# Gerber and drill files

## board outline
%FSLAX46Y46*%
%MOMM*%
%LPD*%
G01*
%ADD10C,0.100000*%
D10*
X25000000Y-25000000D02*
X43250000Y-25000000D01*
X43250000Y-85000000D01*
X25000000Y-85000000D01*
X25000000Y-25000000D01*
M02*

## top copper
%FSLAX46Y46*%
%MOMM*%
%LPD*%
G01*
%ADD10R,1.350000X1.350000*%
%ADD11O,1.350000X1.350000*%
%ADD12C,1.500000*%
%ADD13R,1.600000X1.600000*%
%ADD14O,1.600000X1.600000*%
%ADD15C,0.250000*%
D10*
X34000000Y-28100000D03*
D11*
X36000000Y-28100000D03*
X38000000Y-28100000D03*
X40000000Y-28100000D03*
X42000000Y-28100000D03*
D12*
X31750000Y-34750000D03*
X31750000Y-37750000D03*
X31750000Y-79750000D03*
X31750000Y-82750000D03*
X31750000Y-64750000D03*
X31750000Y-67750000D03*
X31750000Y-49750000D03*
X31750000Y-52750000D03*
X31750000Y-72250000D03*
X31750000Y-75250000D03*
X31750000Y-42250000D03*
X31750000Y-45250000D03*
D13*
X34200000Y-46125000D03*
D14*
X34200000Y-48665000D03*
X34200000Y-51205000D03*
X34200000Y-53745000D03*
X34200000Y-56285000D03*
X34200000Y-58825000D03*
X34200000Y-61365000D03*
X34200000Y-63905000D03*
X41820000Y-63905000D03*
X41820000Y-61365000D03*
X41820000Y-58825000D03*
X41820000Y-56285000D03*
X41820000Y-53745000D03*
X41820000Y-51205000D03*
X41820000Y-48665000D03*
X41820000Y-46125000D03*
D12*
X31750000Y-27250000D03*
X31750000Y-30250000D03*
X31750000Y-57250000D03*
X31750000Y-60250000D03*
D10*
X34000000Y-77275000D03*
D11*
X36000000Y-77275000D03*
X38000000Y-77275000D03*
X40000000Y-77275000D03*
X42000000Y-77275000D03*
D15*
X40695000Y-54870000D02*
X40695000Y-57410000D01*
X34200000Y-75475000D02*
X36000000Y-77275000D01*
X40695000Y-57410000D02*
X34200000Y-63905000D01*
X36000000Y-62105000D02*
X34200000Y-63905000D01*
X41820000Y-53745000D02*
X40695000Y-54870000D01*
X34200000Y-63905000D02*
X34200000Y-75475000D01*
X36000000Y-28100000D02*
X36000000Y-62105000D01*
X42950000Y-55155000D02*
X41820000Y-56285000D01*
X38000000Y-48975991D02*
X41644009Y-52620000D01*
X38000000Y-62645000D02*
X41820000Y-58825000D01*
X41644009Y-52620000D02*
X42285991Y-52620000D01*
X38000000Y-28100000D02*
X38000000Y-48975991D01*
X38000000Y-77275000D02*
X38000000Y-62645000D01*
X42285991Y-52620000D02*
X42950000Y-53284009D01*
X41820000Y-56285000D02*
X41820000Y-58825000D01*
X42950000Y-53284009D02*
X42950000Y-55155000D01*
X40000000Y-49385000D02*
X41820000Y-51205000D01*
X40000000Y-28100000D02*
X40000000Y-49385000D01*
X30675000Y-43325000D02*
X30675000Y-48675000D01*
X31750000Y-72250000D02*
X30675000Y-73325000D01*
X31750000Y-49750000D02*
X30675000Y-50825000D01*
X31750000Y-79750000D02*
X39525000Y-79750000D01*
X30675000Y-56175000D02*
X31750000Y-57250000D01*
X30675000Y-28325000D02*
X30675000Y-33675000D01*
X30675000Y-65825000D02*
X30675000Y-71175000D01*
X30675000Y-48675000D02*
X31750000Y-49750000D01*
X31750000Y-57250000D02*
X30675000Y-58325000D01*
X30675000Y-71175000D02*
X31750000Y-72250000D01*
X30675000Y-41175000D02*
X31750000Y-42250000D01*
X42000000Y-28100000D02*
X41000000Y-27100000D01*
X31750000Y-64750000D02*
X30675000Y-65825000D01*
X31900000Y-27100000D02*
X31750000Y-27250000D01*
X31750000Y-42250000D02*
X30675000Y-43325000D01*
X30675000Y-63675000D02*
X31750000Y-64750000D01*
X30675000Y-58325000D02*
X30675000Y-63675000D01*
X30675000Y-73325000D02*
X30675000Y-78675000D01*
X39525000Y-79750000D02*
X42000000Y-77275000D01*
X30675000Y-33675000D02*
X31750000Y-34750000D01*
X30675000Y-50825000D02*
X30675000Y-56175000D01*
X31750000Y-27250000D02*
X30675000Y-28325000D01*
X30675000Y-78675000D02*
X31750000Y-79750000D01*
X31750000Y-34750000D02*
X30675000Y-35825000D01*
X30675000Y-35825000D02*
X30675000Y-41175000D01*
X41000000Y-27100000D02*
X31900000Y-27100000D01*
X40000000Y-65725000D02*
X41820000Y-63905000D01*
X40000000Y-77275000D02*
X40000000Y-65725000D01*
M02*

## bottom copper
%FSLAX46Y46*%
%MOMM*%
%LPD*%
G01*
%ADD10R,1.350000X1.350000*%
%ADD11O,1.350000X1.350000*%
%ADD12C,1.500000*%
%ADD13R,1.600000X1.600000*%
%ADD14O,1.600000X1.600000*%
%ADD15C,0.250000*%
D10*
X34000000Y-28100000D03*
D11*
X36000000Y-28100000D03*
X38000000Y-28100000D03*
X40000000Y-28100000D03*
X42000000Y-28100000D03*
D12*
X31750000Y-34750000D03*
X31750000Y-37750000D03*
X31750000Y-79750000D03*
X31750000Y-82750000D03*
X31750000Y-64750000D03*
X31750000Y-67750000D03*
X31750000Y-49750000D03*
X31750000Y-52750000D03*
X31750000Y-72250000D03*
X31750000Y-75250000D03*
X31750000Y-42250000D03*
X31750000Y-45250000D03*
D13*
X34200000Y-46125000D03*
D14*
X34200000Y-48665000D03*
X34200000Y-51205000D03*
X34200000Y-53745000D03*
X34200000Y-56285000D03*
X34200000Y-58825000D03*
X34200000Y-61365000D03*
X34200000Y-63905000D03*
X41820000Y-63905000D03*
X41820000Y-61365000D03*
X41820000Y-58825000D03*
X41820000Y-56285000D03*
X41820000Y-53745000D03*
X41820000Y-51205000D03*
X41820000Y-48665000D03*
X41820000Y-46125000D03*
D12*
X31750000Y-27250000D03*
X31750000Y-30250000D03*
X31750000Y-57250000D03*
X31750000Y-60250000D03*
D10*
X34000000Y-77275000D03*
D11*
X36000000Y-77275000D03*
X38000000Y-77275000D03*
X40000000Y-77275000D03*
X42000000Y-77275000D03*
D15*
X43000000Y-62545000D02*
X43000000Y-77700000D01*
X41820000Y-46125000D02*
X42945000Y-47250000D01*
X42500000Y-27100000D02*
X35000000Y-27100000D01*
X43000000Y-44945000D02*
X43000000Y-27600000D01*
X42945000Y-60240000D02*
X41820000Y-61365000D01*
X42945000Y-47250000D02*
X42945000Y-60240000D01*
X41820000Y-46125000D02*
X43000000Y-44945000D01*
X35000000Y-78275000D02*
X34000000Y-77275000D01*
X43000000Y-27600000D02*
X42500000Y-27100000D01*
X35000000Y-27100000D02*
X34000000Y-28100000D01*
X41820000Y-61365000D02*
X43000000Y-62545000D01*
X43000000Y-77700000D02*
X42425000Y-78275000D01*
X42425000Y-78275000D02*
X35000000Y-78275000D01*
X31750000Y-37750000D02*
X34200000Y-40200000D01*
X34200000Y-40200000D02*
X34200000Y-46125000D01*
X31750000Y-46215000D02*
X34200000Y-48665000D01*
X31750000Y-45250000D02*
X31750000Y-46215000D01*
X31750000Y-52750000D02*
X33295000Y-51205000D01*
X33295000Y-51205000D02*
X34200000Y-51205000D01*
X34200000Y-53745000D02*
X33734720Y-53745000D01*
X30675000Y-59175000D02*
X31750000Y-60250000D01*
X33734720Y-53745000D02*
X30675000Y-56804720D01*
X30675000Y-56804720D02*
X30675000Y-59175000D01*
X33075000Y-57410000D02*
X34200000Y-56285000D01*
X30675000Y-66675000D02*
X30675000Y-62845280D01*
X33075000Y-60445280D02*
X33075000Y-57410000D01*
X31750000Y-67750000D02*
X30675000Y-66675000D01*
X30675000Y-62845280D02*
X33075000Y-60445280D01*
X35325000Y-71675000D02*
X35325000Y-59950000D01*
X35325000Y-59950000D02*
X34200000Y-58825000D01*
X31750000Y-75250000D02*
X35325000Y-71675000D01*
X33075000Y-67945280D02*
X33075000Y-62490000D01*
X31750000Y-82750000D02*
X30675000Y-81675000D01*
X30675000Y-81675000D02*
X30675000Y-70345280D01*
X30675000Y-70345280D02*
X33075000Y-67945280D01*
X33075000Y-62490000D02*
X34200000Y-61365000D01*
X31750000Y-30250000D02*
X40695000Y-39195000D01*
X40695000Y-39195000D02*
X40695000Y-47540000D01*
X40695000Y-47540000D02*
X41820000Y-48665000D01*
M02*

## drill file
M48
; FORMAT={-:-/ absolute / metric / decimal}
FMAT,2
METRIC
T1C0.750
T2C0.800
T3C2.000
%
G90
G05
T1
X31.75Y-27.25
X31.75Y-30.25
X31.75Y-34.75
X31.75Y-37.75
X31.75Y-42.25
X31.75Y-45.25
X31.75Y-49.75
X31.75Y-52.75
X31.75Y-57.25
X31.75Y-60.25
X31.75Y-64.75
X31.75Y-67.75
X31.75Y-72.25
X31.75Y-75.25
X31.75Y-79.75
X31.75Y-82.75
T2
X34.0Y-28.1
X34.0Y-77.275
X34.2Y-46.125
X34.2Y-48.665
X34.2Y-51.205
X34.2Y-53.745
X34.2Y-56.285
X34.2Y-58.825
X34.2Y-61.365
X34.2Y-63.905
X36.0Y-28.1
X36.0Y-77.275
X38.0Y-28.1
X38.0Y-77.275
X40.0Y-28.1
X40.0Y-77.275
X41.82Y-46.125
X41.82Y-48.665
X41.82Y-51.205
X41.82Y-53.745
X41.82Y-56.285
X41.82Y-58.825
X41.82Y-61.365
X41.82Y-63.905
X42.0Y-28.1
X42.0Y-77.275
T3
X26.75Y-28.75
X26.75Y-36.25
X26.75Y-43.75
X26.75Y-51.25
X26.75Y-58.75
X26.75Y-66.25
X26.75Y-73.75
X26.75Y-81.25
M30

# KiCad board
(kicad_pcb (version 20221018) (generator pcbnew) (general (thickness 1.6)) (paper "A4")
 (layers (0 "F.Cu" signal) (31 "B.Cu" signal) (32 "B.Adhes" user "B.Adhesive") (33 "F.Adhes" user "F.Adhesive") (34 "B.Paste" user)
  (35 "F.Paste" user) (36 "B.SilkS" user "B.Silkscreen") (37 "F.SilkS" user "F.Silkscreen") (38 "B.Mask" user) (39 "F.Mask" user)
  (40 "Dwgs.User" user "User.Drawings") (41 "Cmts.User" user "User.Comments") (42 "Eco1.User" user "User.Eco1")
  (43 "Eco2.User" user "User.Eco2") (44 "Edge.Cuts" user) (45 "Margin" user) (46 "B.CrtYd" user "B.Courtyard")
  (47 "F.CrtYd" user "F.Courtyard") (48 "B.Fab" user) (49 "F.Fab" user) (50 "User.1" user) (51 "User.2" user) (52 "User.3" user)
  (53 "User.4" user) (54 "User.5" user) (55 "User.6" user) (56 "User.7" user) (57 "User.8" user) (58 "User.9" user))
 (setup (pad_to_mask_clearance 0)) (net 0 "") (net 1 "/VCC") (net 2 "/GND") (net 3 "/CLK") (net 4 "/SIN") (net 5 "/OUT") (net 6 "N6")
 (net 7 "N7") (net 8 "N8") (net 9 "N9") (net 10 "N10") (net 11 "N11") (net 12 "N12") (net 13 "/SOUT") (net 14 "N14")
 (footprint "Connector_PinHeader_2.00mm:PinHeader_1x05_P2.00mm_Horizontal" (layer "F.Cu") (at 34 28.1 90)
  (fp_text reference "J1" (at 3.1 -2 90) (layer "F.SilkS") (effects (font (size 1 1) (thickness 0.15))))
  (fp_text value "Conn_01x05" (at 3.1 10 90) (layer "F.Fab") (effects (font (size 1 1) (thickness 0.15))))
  (pad "1" thru_hole rect (at 0 0 90) (size 1.35 1.35) (drill 0.8) (layers "*.Cu" "*.Mask") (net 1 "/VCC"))
  (pad "2" thru_hole oval (at 0 2 90) (size 1.35 1.35) (drill 0.8) (layers "*.Cu" "*.Mask") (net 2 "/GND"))
  (pad "3" thru_hole oval (at 0 4 90) (size 1.35 1.35) (drill 0.8) (layers "*.Cu" "*.Mask") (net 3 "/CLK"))
  (pad "4" thru_hole oval (at 0 6 90) (size 1.35 1.35) (drill 0.8) (layers "*.Cu" "*.Mask") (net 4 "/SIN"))
  (pad "5" thru_hole oval (at 0 8 90) (size 1.35 1.35) (drill 0.8) (layers "*.Cu" "*.Mask") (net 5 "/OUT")))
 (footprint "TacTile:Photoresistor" (layer "F.Cu") (at 26.75 36.25)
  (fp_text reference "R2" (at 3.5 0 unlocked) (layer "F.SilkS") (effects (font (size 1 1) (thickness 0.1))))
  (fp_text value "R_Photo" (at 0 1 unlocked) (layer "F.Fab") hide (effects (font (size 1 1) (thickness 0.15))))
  (pad "" np_thru_hole circle (at 0 0) (size 2 2) (drill 2) (layers "F&B.Cu" "*.Mask"))
  (pad "1" thru_hole circle (at 5 -1.5) (size 1.5 1.5) (drill 0.75) (layers "*.Cu" "*.Mask") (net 5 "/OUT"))
  (pad "2" thru_hole circle (at 5 1.5) (size 1.5 1.5) (drill 0.75) (layers "*.Cu" "*.Mask") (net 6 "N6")))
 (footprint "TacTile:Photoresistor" (layer "F.Cu") (at 26.75 81.25)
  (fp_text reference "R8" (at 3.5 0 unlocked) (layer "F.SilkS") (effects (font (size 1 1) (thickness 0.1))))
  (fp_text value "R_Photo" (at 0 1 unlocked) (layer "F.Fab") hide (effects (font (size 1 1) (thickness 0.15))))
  (pad "" np_thru_hole circle (at 0 0) (size 2 2) (drill 2) (layers "F&B.Cu" "*.Mask"))
  (pad "1" thru_hole circle (at 5 -1.5) (size 1.5 1.5) (drill 0.75) (layers "*.Cu" "*.Mask") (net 5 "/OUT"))
  (pad "2" thru_hole circle (at 5 1.5) (size 1.5 1.5) (drill 0.75) (layers "*.Cu" "*.Mask") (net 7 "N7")))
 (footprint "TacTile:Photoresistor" (layer "F.Cu") (at 26.75 66.25)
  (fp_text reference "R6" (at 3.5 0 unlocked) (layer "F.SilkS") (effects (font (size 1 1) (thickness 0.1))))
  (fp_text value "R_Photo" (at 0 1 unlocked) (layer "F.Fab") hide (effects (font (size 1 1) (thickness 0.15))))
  (pad "" np_thru_hole circle (at 0 0) (size 2 2) (drill 2) (layers "F&B.Cu" "*.Mask"))
  (pad "1" thru_hole circle (at 5 -1.5) (size 1.5 1.5) (drill 0.75) (layers "*.Cu" "*.Mask") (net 5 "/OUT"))
  (pad "2" thru_hole circle (at 5 1.5) (size 1.5 1.5) (drill 0.75) (layers "*.Cu" "*.Mask") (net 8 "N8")))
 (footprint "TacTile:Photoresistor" (layer "F.Cu") (at 26.75 51.25)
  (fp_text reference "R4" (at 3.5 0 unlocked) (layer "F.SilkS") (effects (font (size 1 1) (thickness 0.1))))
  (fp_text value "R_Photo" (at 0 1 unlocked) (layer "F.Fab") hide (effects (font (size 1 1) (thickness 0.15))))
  (pad "" np_thru_hole circle (at 0 0) (size 2 2) (drill 2) (layers "F&B.Cu" "*.Mask"))
  (pad "1" thru_hole circle (at 5 -1.5) (size 1.5 1.5) (drill 0.75) (layers "*.Cu" "*.Mask") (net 5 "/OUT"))
  (pad "2" thru_hole circle (at 5 1.5) (size 1.5 1.5) (drill 0.75) (layers "*.Cu" "*.Mask") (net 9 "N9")))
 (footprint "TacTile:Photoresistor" (layer "F.Cu") (at 26.75 73.75)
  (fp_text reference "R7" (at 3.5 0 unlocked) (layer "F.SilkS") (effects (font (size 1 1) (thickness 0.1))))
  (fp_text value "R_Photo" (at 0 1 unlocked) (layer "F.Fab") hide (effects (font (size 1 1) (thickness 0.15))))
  (pad "" np_thru_hole circle (at 0 0) (size 2 2) (drill 2) (layers "F&B.Cu" "*.Mask"))
  (pad "1" thru_hole circle (at 5 -1.5) (size 1.5 1.5) (drill 0.75) (layers "*.Cu" "*.Mask") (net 5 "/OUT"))
  (pad "2" thru_hole circle (at 5 1.5) (size 1.5 1.5) (drill 0.75) (layers "*.Cu" "*.Mask") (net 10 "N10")))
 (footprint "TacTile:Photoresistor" (layer "F.Cu") (at 26.75 43.75)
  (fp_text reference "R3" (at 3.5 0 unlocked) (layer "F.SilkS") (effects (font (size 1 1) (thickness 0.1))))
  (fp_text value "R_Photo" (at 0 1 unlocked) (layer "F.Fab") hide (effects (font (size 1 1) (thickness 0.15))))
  (pad "" np_thru_hole circle (at 0 0) (size 2 2) (drill 2) (layers "F&B.Cu" "*.Mask"))
  (pad "1" thru_hole circle (at 5 -1.5) (size 1.5 1.5) (drill 0.75) (layers "*.Cu" "*.Mask") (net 5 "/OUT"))
  (pad "2" thru_hole circle (at 5 1.5) (size 1.5 1.5) (drill 0.75) (layers "*.Cu" "*.Mask") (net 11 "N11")))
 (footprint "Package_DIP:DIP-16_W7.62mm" (layer "F.Cu") (at 34.2 46.125)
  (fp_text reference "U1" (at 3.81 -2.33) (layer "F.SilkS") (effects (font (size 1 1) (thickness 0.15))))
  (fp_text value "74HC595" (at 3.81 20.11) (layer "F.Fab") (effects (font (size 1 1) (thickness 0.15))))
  (pad "1" thru_hole rect (at 0 0) (size 1.6 1.6) (drill 0.8) (layers "*.Cu" "*.Mask") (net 6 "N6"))
  (pad "2" thru_hole oval (at 0 2.54) (size 1.6 1.6) (drill 0.8) (layers "*.Cu" "*.Mask") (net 11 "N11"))
  (pad "3" thru_hole oval (at 0 5.08) (size 1.6 1.6) (drill 0.8) (layers "*.Cu" "*.Mask") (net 9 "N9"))
  (pad "4" thru_hole oval (at 0 7.62) (size 1.6 1.6) (drill 0.8) (layers "*.Cu" "*.Mask") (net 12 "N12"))
  (pad "5" thru_hole oval (at 0 10.16) (size 1.6 1.6) (drill 0.8) (layers "*.Cu" "*.Mask") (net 8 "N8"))
  (pad "6" thru_hole oval (at 0 12.7) (size 1.6 1.6) (drill 0.8) (layers "*.Cu" "*.Mask") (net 10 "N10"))
  (pad "7" thru_hole oval (at 0 15.24) (size 1.6 1.6) (drill 0.8) (layers "*.Cu" "*.Mask") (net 7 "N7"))
  (pad "8" thru_hole oval (at 0 17.78) (size 1.6 1.6) (drill 0.8) (layers "*.Cu" "*.Mask") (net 2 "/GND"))
  (pad "9" thru_hole oval (at 7.62 17.78) (size 1.6 1.6) (drill 0.8) (layers "*.Cu" "*.Mask") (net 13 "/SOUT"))
  (pad "10" thru_hole oval (at 7.62 15.24) (size 1.6 1.6) (drill 0.8) (layers "*.Cu" "*.Mask") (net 1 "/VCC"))
  (pad "11" thru_hole oval (at 7.62 12.7) (size 1.6 1.6) (drill 0.8) (layers "*.Cu" "*.Mask") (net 3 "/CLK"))
  (pad "12" thru_hole oval (at 7.62 10.16) (size 1.6 1.6) (drill 0.8) (layers "*.Cu" "*.Mask") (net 3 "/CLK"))
  (pad "13" thru_hole oval (at 7.62 7.62) (size 1.6 1.6) (drill 0.8) (layers "*.Cu" "*.Mask") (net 2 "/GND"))
  (pad "14" thru_hole oval (at 7.62 5.08) (size 1.6 1.6) (drill 0.8) (layers "*.Cu" "*.Mask") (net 4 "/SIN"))
  (pad "15" thru_hole oval (at 7.62 2.54) (size 1.6 1.6) (drill 0.8) (layers "*.Cu" "*.Mask") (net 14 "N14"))
  (pad "16" thru_hole oval (at 7.62 0) (size 1.6 1.6) (drill 0.8) (layers "*.Cu" "*.Mask") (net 1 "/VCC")))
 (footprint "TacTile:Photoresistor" (layer "F.Cu") (at 26.75 28.75)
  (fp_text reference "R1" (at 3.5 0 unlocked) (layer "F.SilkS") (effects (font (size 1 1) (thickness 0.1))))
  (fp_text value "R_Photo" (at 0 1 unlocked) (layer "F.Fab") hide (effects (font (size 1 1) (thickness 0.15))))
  (pad "" np_thru_hole circle (at 0 0) (size 2 2) (drill 2) (layers "F&B.Cu" "*.Mask"))
  (pad "1" thru_hole circle (at 5 -1.5) (size 1.5 1.5) (drill 0.75) (layers "*.Cu" "*.Mask") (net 5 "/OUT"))
  (pad "2" thru_hole circle (at 5 1.5) (size 1.5 1.5) (drill 0.75) (layers "*.Cu" "*.Mask") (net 14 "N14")))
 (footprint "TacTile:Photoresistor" (layer "F.Cu") (at 26.75 58.75)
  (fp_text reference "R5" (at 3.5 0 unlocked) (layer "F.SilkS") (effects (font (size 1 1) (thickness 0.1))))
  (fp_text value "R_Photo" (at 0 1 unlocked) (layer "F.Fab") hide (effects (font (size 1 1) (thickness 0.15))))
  (pad "" np_thru_hole circle (at 0 0) (size 2 2) (drill 2) (layers "F&B.Cu" "*.Mask"))
  (pad "1" thru_hole circle (at 5 -1.5) (size 1.5 1.5) (drill 0.75) (layers "*.Cu" "*.Mask") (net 5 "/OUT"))
  (pad "2" thru_hole circle (at 5 1.5) (size 1.5 1.5) (drill 0.75) (layers "*.Cu" "*.Mask") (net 12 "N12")))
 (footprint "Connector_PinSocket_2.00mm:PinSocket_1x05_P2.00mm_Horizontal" (layer "F.Cu") (at 34 77.275 90)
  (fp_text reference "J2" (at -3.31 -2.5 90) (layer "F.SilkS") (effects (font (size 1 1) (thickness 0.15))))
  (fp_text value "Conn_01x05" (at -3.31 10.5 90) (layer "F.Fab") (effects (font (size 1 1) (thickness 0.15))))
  (pad "1" thru_hole rect (at 0 0 90) (size 1.35 1.35) (drill 0.8) (layers "*.Cu" "*.Mask") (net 1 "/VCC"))
  (pad "2" thru_hole oval (at 0 2 90) (size 1.35 1.35) (drill 0.8) (layers "*.Cu" "*.Mask") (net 2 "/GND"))
  (pad "3" thru_hole oval (at 0 4 90) (size 1.35 1.35) (drill 0.8) (layers "*.Cu" "*.Mask") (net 3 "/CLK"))
  (pad "4" thru_hole oval (at 0 6 90) (size 1.35 1.35) (drill 0.8) (layers "*.Cu" "*.Mask") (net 13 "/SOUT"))
  (pad "5" thru_hole oval (at 0 8 90) (size 1.35 1.35) (drill 0.8) (layers "*.Cu" "*.Mask") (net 5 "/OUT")))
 (gr_rect (start 25 25) (end 43.25 85) (stroke (width 0.1) (type default)) (fill none) (layer "Edge.Cuts"))
 (segment (start 43 62.545) (end 43 77.7) (width 0.25) (layer "B.Cu") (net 1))
 (segment (start 41.82 46.125) (end 42.945 47.25) (width 0.25) (layer "B.Cu") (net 1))
 (segment (start 42.5 27.1) (end 35 27.1) (width 0.25) (layer "B.Cu") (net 1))
 (segment (start 43 44.945) (end 43 27.6) (width 0.25) (layer "B.Cu") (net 1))
 (segment (start 42.945 60.24) (end 41.82 61.365) (width 0.25) (layer "B.Cu") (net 1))
 (segment (start 42.945 47.25) (end 42.945 60.24) (width 0.25) (layer "B.Cu") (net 1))
 (segment (start 41.82 46.125) (end 43 44.945) (width 0.25) (layer "B.Cu") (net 1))
 (segment (start 35 78.275) (end 34 77.275) (width 0.25) (layer "B.Cu") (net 1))
 (segment (start 43 27.6) (end 42.5 27.1) (width 0.25) (layer "B.Cu") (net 1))
 (segment (start 35 27.1) (end 34 28.1) (width 0.25) (layer "B.Cu") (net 1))
 (segment (start 41.82 61.365) (end 43 62.545) (width 0.25) (layer "B.Cu") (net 1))
 (segment (start 43 77.7) (end 42.425 78.275) (width 0.25) (layer "B.Cu") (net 1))
 (segment (start 42.425 78.275) (end 35 78.275) (width 0.25) (layer "B.Cu") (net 1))
 (segment (start 40.695 54.87) (end 40.695 57.41) (width 0.25) (layer "F.Cu") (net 2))
 (segment (start 34.2 75.475) (end 36 77.275) (width 0.25) (layer "F.Cu") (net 2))
 (segment (start 40.695 57.41) (end 34.2 63.905) (width 0.25) (layer "F.Cu") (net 2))
 (segment (start 36 62.105) (end 34.2 63.905) (width 0.25) (layer "F.Cu") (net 2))
 (segment (start 41.82 53.745) (end 40.695 54.87) (width 0.25) (layer "F.Cu") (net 2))
 (segment (start 34.2 63.905) (end 34.2 75.475) (width 0.25) (layer "F.Cu") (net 2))
 (segment (start 36 28.1) (end 36 62.105) (width 0.25) (layer "F.Cu") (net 2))
 (segment (start 42.95 55.155) (end 41.82 56.285) (width 0.25) (layer "F.Cu") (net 3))
 (segment (start 38 48.975991) (end 41.644009 52.62) (width 0.25) (layer "F.Cu") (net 3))
 (segment (start 38 62.645) (end 41.82 58.825) (width 0.25) (layer "F.Cu") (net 3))
 (segment (start 41.644009 52.62) (end 42.285991 52.62) (width 0.25) (layer "F.Cu") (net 3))
 (segment (start 38 28.1) (end 38 48.975991) (width 0.25) (layer "F.Cu") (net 3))
 (segment (start 38 77.275) (end 38 62.645) (width 0.25) (layer "F.Cu") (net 3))
 (segment (start 42.285991 52.62) (end 42.95 53.284009) (width 0.25) (layer "F.Cu") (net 3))
 (segment (start 41.82 56.285) (end 41.82 58.825) (width 0.25) (layer "F.Cu") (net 3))
 (segment (start 42.95 53.284009) (end 42.95 55.155) (width 0.25) (layer "F.Cu") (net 3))
 (segment (start 40 49.385) (end 41.82 51.205) (width 0.25) (layer "F.Cu") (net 4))
 (segment (start 40 28.1) (end 40 49.385) (width 0.25) (layer "F.Cu") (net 4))
 (segment (start 30.675 43.325) (end 30.675 48.675) (width 0.25) (layer "F.Cu") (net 5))
 (segment (start 31.75 72.25) (end 30.675 73.325) (width 0.25) (layer "F.Cu") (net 5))
 (segment (start 31.75 49.75) (end 30.675 50.825) (width 0.25) (layer "F.Cu") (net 5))
 (segment (start 31.75 79.75) (end 39.525 79.75) (width 0.25) (layer "F.Cu") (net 5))
 (segment (start 30.675 56.175) (end 31.75 57.25) (width 0.25) (layer "F.Cu") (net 5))
 (segment (start 30.675 28.325) (end 30.675 33.675) (width 0.25) (layer "F.Cu") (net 5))
 (segment (start 30.675 65.825) (end 30.675 71.175) (width 0.25) (layer "F.Cu") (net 5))
 (segment (start 30.675 48.675) (end 31.75 49.75) (width 0.25) (layer "F.Cu") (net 5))
 (segment (start 31.75 57.25) (end 30.675 58.325) (width 0.25) (layer "F.Cu") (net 5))
 (segment (start 30.675 71.175) (end 31.75 72.25) (width 0.25) (layer "F.Cu") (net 5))
 (segment (start 30.675 41.175) (end 31.75 42.25) (width 0.25) (layer "F.Cu") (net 5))
 (segment (start 42 28.1) (end 41 27.1) (width 0.25) (layer "F.Cu") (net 5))
 (segment (start 31.75 64.75) (end 30.675 65.825) (width 0.25) (layer "F.Cu") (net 5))
 (segment (start 31.9 27.1) (end 31.75 27.25) (width 0.25) (layer "F.Cu") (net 5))
 (segment (start 31.75 42.25) (end 30.675 43.325) (width 0.25) (layer "F.Cu") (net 5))
 (segment (start 30.675 63.675) (end 31.75 64.75) (width 0.25) (layer "F.Cu") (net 5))
 (segment (start 30.675 58.325) (end 30.675 63.675) (width 0.25) (layer "F.Cu") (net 5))
 (segment (start 30.675 73.325) (end 30.675 78.675) (width 0.25) (layer "F.Cu") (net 5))
 (segment (start 39.525 79.75) (end 42 77.275) (width 0.25) (layer "F.Cu") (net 5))
 (segment (start 30.675 33.675) (end 31.75 34.75) (width 0.25) (layer "F.Cu") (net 5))
 (segment (start 30.675 50.825) (end 30.675 56.175) (width 0.25) (layer "F.Cu") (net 5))
 (segment (start 31.75 27.25) (end 30.675 28.325) (width 0.25) (layer "F.Cu") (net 5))
 (segment (start 30.675 78.675) (end 31.75 79.75) (width 0.25) (layer "F.Cu") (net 5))
 (segment (start 31.75 34.75) (end 30.675 35.825) (width 0.25) (layer "F.Cu") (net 5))
 (segment (start 30.675 35.825) (end 30.675 41.175) (width 0.25) (layer "F.Cu") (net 5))
 (segment (start 41 27.1) (end 31.9 27.1) (width 0.25) (layer "F.Cu") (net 5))
 (segment (start 40 65.725) (end 41.82 63.905) (width 0.25) (layer "F.Cu") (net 13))
 (segment (start 40 77.275) (end 40 65.725) (width 0.25) (layer "F.Cu") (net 13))
 (segment (start 31.75 37.75) (end 34.2 40.2) (width 0.25) (layer "B.Cu") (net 6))
 (segment (start 34.2 40.2) (end 34.2 46.125) (width 0.25) (layer "B.Cu") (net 6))
 (segment (start 31.75 46.215) (end 34.2 48.665) (width 0.25) (layer "B.Cu") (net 11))
 (segment (start 31.75 45.25) (end 31.75 46.215) (width 0.25) (layer "B.Cu") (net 11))
 (segment (start 31.75 52.75) (end 33.295 51.205) (width 0.25) (layer "B.Cu") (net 9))
 (segment (start 33.295 51.205) (end 34.2 51.205) (width 0.25) (layer "B.Cu") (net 9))
 (segment (start 34.2 53.745) (end 33.73472 53.745) (width 0.25) (layer "B.Cu") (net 12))
 (segment (start 30.675 59.175) (end 31.75 60.25) (width 0.25) (layer "B.Cu") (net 12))
 (segment (start 33.73472 53.745) (end 30.675 56.80472) (width 0.25) (layer "B.Cu") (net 12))
 (segment (start 30.675 56.80472) (end 30.675 59.175) (width 0.25) (layer "B.Cu") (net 12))
 (segment (start 33.075 57.41) (end 34.2 56.285) (width 0.25) (layer "B.Cu") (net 8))
 (segment (start 30.675 66.675) (end 30.675 62.84528) (width 0.25) (layer "B.Cu") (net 8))
 (segment (start 33.075 60.44528) (end 33.075 57.41) (width 0.25) (layer "B.Cu") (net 8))
 (segment (start 31.75 67.75) (end 30.675 66.675) (width 0.25) (layer "B.Cu") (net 8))
 (segment (start 30.675 62.84528) (end 33.075 60.44528) (width 0.25) (layer "B.Cu") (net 8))
 (segment (start 35.325 71.675) (end 35.325 59.95) (width 0.25) (layer "B.Cu") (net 10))
 (segment (start 35.325 59.95) (end 34.2 58.825) (width 0.25) (layer "B.Cu") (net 10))
 (segment (start 31.75 75.25) (end 35.325 71.675) (width 0.25) (layer "B.Cu") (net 10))
 (segment (start 33.075 67.94528) (end 33.075 62.49) (width 0.25) (layer "B.Cu") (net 7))
 (segment (start 31.75 82.75) (end 30.675 81.675) (width 0.25) (layer "B.Cu") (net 7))
 (segment (start 30.675 81.675) (end 30.675 70.34528) (width 0.25) (layer "B.Cu") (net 7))
 (segment (start 30.675 70.34528) (end 33.075 67.94528) (width 0.25) (layer "B.Cu") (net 7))
 (segment (start 33.075 62.49) (end 34.2 61.365) (width 0.25) (layer "B.Cu") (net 7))
 (segment (start 31.75 30.25) (end 40.695 39.195) (width 0.25) (layer "B.Cu") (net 14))
 (segment (start 40.695 39.195) (end 40.695 47.54) (width 0.25) (layer "B.Cu") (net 14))
 (segment (start 40.695 47.54) (end 41.82 48.665) (width 0.25) (layer "B.Cu") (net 14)))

